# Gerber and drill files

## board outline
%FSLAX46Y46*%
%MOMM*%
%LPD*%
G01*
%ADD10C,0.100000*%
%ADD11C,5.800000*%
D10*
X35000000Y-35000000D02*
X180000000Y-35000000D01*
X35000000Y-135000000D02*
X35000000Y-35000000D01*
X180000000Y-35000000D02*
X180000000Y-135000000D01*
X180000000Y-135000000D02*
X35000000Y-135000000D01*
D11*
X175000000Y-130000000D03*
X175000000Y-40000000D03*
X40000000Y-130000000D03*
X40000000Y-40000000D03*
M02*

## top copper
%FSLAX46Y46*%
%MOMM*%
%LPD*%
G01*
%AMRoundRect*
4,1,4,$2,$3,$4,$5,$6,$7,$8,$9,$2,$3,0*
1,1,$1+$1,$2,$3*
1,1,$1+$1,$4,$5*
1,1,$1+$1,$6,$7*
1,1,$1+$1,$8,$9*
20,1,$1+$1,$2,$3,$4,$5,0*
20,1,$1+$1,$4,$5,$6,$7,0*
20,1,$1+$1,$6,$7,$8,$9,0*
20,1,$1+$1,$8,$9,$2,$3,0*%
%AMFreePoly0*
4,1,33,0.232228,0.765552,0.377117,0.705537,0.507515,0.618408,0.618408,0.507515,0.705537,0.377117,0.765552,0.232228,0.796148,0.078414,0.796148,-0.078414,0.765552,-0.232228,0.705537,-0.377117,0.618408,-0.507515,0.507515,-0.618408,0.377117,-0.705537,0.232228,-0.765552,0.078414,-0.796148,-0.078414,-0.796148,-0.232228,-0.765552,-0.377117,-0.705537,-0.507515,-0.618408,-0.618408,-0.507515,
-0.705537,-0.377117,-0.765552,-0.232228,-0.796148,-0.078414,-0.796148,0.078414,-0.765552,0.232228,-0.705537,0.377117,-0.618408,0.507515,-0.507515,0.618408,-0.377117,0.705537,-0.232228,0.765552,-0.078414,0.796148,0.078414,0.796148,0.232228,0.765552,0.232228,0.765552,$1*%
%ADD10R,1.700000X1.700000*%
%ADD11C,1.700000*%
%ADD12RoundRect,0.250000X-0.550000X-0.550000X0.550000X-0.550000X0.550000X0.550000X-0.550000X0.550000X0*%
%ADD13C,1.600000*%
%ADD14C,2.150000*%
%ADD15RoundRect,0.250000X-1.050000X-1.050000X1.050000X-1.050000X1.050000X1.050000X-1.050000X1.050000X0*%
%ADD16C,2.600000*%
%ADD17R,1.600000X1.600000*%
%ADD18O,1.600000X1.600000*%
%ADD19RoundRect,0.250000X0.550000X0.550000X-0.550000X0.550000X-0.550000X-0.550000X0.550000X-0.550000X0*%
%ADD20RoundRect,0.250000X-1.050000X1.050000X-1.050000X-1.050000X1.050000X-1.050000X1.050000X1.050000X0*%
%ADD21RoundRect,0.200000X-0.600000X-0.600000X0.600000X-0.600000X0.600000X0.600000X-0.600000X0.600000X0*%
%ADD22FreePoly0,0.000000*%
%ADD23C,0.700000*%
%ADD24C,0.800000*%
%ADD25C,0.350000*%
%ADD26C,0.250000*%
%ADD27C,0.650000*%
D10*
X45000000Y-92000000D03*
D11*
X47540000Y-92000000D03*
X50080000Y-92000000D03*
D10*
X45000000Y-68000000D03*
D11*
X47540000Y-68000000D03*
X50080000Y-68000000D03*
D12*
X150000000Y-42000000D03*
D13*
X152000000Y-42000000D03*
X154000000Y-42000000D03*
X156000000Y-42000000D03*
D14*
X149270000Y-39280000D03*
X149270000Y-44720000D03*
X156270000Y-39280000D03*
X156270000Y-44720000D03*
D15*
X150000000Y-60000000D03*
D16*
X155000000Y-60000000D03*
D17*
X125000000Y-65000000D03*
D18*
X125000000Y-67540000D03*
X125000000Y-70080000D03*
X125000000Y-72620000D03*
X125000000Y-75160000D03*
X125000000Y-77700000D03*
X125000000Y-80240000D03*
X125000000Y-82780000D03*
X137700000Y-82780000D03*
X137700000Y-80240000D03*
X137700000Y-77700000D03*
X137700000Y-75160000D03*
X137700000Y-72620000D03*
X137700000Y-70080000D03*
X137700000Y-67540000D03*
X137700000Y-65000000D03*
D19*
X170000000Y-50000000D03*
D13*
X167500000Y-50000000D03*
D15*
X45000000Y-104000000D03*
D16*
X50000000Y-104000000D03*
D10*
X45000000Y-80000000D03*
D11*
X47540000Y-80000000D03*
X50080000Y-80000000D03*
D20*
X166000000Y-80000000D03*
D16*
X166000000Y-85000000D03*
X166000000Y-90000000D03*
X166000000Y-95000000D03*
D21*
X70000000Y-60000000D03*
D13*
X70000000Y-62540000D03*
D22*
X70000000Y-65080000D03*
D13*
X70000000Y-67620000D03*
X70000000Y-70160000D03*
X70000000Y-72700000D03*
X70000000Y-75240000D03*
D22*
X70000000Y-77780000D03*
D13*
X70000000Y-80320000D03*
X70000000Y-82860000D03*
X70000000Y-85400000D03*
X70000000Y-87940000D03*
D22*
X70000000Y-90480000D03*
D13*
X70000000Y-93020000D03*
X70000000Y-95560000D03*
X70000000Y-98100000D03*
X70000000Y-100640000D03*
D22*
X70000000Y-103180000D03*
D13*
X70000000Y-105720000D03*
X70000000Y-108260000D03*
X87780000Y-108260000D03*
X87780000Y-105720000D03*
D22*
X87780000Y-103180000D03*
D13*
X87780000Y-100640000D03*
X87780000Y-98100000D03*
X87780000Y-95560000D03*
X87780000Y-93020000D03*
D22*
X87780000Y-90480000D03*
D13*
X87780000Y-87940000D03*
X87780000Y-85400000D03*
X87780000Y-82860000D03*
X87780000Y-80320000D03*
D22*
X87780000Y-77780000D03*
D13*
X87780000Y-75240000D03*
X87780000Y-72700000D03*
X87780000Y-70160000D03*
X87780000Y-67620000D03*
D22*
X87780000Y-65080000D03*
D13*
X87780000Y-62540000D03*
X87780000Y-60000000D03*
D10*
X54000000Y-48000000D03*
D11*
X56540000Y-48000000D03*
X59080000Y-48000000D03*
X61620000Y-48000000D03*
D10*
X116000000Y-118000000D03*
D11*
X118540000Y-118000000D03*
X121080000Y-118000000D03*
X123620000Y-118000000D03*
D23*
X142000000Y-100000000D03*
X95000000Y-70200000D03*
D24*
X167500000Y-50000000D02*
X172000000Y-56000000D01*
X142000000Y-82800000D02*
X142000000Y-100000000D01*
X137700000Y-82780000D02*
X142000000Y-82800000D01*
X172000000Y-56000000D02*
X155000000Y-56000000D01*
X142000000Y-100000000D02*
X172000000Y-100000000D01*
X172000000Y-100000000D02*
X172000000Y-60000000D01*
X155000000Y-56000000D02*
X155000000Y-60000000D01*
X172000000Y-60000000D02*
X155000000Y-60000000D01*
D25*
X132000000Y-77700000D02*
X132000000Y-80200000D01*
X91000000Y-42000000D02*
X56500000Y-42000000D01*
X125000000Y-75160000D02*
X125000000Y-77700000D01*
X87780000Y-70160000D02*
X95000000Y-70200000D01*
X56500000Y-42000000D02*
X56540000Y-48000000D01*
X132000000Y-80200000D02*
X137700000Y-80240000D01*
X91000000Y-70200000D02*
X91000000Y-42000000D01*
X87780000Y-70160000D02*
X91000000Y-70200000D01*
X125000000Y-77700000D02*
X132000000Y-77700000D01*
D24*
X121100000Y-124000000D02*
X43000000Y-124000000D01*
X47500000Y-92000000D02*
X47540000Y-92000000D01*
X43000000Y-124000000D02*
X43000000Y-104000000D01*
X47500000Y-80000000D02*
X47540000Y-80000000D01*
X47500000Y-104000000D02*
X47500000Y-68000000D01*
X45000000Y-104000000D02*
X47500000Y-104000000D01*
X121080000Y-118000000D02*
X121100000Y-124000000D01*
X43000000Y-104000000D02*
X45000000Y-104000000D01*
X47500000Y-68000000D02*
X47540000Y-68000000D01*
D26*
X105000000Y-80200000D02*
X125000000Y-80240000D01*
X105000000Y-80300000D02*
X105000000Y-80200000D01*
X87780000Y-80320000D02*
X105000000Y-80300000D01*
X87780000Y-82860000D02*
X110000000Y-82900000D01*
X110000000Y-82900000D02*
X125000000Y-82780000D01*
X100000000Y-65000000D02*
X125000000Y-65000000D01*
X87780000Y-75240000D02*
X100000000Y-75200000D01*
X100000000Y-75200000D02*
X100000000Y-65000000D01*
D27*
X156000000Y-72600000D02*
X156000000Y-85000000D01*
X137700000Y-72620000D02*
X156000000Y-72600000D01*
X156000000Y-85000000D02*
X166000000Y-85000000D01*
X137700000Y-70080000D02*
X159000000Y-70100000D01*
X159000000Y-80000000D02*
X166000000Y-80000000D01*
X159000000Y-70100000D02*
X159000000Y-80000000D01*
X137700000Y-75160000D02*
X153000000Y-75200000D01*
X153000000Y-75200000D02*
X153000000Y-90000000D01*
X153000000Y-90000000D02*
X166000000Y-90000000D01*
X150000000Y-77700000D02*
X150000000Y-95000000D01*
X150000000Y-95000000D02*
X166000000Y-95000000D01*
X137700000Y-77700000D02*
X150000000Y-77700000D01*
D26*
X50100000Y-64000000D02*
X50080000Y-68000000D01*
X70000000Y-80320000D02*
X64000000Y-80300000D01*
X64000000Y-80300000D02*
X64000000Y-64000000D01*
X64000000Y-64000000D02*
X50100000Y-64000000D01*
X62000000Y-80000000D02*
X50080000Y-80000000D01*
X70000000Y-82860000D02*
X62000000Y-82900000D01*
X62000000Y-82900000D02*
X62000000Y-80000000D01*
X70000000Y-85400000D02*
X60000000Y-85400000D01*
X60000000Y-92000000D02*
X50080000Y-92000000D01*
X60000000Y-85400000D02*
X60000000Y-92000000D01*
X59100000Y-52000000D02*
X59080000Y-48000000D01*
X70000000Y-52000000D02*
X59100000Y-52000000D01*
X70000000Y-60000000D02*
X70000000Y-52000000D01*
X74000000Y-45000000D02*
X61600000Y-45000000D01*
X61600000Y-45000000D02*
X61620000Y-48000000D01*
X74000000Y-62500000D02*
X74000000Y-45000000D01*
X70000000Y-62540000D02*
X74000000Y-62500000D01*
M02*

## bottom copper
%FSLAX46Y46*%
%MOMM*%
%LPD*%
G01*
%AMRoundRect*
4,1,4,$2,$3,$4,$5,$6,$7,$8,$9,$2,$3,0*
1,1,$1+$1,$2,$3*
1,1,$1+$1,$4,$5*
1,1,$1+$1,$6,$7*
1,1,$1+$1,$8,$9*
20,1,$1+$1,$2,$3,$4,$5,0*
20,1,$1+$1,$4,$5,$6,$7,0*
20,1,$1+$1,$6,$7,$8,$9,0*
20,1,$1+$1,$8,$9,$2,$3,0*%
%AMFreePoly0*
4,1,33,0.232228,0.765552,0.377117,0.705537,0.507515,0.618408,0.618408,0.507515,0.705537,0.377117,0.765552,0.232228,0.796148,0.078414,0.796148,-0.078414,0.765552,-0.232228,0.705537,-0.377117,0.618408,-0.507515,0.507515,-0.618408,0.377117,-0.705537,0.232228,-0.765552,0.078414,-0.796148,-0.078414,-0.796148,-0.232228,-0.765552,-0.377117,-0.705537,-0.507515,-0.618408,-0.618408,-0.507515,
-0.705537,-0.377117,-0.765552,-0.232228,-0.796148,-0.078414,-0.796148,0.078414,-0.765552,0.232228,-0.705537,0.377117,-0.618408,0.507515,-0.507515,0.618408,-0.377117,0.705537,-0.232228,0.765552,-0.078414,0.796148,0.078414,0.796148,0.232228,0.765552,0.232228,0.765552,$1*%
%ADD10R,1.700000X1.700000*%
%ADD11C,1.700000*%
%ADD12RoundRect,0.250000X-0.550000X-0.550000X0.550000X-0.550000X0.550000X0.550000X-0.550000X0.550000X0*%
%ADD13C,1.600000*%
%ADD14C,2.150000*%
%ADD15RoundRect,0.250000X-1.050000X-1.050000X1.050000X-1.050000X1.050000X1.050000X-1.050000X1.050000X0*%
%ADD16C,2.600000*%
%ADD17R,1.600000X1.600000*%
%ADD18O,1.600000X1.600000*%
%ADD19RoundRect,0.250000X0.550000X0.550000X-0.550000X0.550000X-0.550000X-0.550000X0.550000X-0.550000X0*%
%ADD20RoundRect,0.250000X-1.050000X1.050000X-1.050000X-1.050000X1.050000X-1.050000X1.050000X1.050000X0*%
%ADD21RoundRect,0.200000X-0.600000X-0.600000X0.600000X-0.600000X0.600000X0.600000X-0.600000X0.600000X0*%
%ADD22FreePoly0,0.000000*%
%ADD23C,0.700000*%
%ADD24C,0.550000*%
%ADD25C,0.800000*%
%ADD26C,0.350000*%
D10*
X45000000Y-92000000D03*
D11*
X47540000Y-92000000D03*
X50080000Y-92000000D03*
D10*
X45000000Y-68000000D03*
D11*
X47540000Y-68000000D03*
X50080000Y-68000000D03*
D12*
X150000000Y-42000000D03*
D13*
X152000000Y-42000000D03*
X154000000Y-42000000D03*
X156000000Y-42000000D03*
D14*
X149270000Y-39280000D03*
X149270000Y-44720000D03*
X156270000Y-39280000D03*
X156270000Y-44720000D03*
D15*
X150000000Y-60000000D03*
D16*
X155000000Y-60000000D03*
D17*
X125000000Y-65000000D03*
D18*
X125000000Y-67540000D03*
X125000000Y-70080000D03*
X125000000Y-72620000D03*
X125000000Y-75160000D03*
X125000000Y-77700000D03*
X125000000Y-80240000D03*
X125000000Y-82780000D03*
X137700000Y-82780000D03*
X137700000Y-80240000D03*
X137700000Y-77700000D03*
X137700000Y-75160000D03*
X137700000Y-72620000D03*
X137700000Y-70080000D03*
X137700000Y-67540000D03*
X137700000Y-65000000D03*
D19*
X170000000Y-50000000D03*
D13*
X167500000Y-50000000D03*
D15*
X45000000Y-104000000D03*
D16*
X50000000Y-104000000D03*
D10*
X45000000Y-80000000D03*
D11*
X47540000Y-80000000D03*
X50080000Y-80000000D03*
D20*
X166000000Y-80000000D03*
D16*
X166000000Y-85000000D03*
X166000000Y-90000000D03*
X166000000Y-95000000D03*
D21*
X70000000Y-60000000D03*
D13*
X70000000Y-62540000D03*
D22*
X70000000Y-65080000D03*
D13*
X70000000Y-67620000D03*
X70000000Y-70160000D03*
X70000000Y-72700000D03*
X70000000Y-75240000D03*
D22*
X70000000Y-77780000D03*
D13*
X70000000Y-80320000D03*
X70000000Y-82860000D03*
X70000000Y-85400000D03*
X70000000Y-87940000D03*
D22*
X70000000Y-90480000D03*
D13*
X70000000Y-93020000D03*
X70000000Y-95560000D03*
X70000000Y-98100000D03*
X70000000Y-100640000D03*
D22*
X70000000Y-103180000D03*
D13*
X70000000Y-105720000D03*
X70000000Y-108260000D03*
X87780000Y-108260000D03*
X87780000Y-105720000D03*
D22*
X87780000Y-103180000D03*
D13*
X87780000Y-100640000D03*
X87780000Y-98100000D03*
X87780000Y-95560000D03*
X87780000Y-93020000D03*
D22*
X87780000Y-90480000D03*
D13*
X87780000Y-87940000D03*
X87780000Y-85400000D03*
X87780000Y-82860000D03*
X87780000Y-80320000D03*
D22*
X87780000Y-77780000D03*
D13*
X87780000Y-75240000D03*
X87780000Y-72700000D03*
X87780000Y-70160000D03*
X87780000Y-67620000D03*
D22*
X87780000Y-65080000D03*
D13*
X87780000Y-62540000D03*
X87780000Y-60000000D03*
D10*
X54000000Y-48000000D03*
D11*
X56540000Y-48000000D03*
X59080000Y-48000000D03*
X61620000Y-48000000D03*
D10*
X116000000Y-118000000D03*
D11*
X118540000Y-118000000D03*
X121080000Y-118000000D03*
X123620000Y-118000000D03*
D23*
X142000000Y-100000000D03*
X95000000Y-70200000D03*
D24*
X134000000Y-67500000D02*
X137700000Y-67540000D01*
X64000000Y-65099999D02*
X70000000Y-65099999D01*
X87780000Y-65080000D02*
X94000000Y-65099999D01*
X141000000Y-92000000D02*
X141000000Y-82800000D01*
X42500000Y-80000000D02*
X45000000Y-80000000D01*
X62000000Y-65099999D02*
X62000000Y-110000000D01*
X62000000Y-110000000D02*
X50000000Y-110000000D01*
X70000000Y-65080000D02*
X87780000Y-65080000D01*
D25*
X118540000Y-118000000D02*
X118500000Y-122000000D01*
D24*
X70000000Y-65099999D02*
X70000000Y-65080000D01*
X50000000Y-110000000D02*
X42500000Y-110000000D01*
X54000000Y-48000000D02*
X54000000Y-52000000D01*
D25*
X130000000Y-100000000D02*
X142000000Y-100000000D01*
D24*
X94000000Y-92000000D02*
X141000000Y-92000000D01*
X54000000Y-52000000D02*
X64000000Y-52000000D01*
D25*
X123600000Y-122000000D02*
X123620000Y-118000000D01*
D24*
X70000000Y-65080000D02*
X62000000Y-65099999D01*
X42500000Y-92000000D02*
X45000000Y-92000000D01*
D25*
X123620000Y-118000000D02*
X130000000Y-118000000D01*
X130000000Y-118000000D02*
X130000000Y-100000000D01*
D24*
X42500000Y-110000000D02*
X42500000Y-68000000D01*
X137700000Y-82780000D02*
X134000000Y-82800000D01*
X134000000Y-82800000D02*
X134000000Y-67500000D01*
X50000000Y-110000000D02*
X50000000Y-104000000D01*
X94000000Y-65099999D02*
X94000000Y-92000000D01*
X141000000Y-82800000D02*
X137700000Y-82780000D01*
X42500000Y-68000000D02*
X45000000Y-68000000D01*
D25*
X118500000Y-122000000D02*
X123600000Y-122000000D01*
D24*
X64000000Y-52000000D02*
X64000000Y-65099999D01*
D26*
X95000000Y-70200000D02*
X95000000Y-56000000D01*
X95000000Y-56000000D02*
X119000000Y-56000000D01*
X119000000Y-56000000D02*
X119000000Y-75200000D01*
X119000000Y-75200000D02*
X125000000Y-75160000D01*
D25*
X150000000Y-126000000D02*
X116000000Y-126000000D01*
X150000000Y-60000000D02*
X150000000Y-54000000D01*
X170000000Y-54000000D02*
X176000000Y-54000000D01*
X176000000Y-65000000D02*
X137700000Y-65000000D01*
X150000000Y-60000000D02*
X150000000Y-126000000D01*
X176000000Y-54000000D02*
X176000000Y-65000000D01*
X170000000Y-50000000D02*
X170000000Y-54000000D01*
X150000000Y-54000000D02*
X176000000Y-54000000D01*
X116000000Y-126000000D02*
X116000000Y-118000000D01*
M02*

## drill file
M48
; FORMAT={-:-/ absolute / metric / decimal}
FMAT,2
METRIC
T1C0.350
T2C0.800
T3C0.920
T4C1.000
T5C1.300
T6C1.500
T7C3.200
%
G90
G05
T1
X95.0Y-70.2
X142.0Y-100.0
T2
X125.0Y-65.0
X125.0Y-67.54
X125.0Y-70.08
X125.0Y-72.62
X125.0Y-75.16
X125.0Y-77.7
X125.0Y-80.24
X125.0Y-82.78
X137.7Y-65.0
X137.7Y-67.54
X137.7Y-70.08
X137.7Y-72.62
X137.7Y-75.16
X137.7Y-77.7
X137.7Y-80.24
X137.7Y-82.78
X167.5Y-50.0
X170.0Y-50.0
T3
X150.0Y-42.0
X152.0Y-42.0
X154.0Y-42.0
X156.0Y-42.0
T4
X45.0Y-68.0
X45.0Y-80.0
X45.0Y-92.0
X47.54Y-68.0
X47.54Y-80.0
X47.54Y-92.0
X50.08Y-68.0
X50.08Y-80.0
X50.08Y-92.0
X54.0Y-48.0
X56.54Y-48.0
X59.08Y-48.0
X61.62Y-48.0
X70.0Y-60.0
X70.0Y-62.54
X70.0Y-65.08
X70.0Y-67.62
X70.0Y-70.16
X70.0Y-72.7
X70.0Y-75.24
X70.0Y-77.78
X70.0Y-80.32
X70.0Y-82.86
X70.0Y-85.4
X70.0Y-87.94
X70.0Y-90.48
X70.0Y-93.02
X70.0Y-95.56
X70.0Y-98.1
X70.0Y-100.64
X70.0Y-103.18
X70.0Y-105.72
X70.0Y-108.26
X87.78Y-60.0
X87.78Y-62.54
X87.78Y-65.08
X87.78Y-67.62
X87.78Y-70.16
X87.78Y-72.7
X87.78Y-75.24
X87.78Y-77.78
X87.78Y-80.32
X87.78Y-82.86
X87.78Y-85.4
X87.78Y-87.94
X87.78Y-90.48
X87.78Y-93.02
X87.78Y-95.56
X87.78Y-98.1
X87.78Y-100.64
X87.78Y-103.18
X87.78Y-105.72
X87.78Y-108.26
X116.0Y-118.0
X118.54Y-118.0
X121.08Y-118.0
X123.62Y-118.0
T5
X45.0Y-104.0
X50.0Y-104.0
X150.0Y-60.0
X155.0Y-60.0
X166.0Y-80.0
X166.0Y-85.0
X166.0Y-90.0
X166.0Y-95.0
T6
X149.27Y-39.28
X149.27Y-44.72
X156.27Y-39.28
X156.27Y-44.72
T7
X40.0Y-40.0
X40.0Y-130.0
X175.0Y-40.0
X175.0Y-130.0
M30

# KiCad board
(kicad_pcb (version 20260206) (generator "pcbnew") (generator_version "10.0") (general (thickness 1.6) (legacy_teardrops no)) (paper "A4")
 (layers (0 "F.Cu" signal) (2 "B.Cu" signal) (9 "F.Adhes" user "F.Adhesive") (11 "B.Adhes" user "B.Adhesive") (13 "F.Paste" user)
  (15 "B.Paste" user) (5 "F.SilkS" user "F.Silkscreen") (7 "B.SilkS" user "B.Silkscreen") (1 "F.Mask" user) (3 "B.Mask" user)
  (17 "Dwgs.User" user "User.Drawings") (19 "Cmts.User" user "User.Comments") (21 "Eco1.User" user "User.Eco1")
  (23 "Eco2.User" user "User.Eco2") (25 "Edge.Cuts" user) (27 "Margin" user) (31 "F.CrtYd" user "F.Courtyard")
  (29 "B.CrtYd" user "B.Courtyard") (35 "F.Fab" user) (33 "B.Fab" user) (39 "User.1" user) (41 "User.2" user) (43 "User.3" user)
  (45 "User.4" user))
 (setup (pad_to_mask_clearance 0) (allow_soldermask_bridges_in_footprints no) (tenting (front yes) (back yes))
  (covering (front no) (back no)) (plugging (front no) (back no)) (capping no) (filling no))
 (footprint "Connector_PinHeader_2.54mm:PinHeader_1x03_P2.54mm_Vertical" (layer "F.Cu") (at 45 92 90)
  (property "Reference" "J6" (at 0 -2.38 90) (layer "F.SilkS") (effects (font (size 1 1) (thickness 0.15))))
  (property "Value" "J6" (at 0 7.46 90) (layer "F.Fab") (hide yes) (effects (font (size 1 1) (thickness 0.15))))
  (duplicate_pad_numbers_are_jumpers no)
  (pad "1" thru_hole rect (at 0 0 90) (size 1.7 1.7) (drill 1) (layers "*.Cu" "*.Mask") (remove_unused_layers no) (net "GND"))
  (pad "2" thru_hole circle (at 0 2.54 90) (size 1.7 1.7) (drill 1) (layers "*.Cu" "*.Mask") (remove_unused_layers no) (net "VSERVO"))
  (pad "3" thru_hole circle (at 0 5.08 90) (size 1.7 1.7) (drill 1) (layers "*.Cu" "*.Mask") (remove_unused_layers no) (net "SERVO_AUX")))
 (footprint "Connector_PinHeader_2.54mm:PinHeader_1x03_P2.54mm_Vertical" (layer "F.Cu") (at 45 68 90)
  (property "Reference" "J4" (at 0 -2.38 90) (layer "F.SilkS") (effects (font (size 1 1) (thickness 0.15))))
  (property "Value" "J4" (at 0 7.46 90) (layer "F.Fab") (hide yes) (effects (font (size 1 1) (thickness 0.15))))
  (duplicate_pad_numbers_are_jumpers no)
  (pad "1" thru_hole rect (at 0 0 90) (size 1.7 1.7) (drill 1) (layers "*.Cu" "*.Mask") (remove_unused_layers no) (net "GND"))
  (pad "2" thru_hole circle (at 0 2.54 90) (size 1.7 1.7) (drill 1) (layers "*.Cu" "*.Mask") (remove_unused_layers no) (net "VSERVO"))
  (pad "3" thru_hole circle (at 0 5.08 90) (size 1.7 1.7) (drill 1) (layers "*.Cu" "*.Mask") (remove_unused_layers no) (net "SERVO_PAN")))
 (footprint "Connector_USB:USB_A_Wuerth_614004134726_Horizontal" (layer "F.Cu") (at 150 42)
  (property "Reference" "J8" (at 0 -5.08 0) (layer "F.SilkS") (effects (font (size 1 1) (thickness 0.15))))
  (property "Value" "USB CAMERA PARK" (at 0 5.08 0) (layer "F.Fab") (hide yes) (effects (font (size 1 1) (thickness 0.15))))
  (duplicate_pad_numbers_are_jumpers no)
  (pad "1" thru_hole roundrect (at 0 0) (size 1.6 1.6) (drill 0.92) (layers "*.Cu" "*.Mask") (remove_unused_layers no)
   (roundrect_rratio 0.15625) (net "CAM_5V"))
  (pad "2" thru_hole circle (at 2 0) (size 1.6 1.6) (drill 0.92) (layers "*.Cu" "*.Mask") (remove_unused_layers no) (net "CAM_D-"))
  (pad "3" thru_hole circle (at 4 0) (size 1.6 1.6) (drill 0.92) (layers "*.Cu" "*.Mask") (remove_unused_layers no) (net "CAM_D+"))
  (pad "4" thru_hole circle (at 6 0) (size 1.6 1.6) (drill 0.92) (layers "*.Cu" "*.Mask") (remove_unused_layers no) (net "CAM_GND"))
  (pad "SH" thru_hole circle (at -0.73 -2.72) (size 2.15 2.15) (drill 1.5) (layers "*.Cu" "*.Mask") (remove_unused_layers no))
  (pad "SH" thru_hole circle (at -0.73 2.72) (size 2.15 2.15) (drill 1.5) (layers "*.Cu" "*.Mask") (remove_unused_layers no))
  (pad "SH" thru_hole circle (at 6.27 -2.72) (size 2.15 2.15) (drill 1.5) (layers "*.Cu" "*.Mask") (remove_unused_layers no))
  (pad "SH" thru_hole circle (at 6.27 2.72) (size 2.15 2.15) (drill 1.5) (layers "*.Cu" "*.Mask") (remove_unused_layers no)))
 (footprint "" (layer "F.Cu") (at 175 130)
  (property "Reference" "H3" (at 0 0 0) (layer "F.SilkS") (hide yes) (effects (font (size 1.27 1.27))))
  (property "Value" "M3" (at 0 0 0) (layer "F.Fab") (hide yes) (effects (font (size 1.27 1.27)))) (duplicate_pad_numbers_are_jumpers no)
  (pad "" np_thru_hole circle (at 0 0) (size 5.8 5.8) (drill 3.2) (layers "Edge.Cuts")))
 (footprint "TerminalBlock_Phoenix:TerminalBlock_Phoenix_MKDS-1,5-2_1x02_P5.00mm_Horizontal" (layer "F.Cu") (at 150 60)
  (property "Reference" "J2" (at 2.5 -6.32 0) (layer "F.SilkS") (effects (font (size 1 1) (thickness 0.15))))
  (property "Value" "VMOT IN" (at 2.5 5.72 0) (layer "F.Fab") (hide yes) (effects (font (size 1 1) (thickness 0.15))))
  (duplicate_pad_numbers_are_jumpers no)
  (pad "1" thru_hole roundrect (at 0 0) (size 2.6 2.6) (drill 1.3) (layers "*.Cu" "*.Mask") (remove_unused_layers no)
   (roundrect_rratio 0.096154) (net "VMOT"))
  (pad "2" thru_hole circle (at 5 0) (size 2.6 2.6) (drill 1.3) (layers "*.Cu" "*.Mask") (remove_unused_layers no) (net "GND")))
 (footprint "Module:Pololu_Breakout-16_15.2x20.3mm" (layer "F.Cu") (at 125 65)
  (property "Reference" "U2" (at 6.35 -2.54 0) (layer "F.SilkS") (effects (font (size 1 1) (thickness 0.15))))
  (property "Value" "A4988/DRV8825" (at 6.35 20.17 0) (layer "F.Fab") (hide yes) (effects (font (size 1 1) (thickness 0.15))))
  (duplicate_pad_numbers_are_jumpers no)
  (pad "1" thru_hole rect (at 0 0) (size 1.6 1.6) (drill 0.8) (layers "*.Cu" "*.Mask") (remove_unused_layers no) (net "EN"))
  (pad "2" thru_hole oval (at 0 2.54) (size 1.6 1.6) (drill 0.8) (layers "*.Cu" "*.Mask") (remove_unused_layers no))
  (pad "3" thru_hole oval (at 0 5.08) (size 1.6 1.6) (drill 0.8) (layers "*.Cu" "*.Mask") (remove_unused_layers no))
  (pad "4" thru_hole oval (at 0 7.62) (size 1.6 1.6) (drill 0.8) (layers "*.Cu" "*.Mask") (remove_unused_layers no))
  (pad "5" thru_hole oval (at 0 10.16) (size 1.6 1.6) (drill 0.8) (layers "*.Cu" "*.Mask") (remove_unused_layers no) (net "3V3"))
  (pad "6" thru_hole oval (at 0 12.7) (size 1.6 1.6) (drill 0.8) (layers "*.Cu" "*.Mask") (remove_unused_layers no) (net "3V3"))
  (pad "7" thru_hole oval (at 0 15.24) (size 1.6 1.6) (drill 0.8) (layers "*.Cu" "*.Mask") (remove_unused_layers no) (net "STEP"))
  (pad "8" thru_hole oval (at 0 17.78) (size 1.6 1.6) (drill 0.8) (layers "*.Cu" "*.Mask") (remove_unused_layers no) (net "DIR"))
  (pad "9" thru_hole oval (at 12.7 17.78) (size 1.6 1.6) (drill 0.8) (layers "*.Cu" "*.Mask") (remove_unused_layers no) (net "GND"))
  (pad "10" thru_hole oval (at 12.7 15.24) (size 1.6 1.6) (drill 0.8) (layers "*.Cu" "*.Mask") (remove_unused_layers no) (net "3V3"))
  (pad "11" thru_hole oval (at 12.7 12.7) (size 1.6 1.6) (drill 0.8) (layers "*.Cu" "*.Mask") (remove_unused_layers no) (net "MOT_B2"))
  (pad "12" thru_hole oval (at 12.7 10.16) (size 1.6 1.6) (drill 0.8) (layers "*.Cu" "*.Mask") (remove_unused_layers no) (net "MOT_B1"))
  (pad "13" thru_hole oval (at 12.7 7.62) (size 1.6 1.6) (drill 0.8) (layers "*.Cu" "*.Mask") (remove_unused_layers no) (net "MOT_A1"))
  (pad "14" thru_hole oval (at 12.7 5.08) (size 1.6 1.6) (drill 0.8) (layers "*.Cu" "*.Mask") (remove_unused_layers no) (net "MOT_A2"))
  (pad "15" thru_hole oval (at 12.7 2.54) (size 1.6 1.6) (drill 0.8) (layers "*.Cu" "*.Mask") (remove_unused_layers no) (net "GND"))
  (pad "16" thru_hole oval (at 12.7 0) (size 1.6 1.6) (drill 0.8) (layers "*.Cu" "*.Mask") (remove_unused_layers no) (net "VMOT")))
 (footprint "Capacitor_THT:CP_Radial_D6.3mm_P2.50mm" (layer "F.Cu") (at 170 50 180)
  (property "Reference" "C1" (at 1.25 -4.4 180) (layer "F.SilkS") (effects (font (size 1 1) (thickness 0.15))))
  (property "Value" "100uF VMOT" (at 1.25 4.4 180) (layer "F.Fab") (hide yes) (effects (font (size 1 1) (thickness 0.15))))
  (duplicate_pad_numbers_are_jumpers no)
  (pad "1" thru_hole roundrect (at 0 0 180) (size 1.6 1.6) (drill 0.8) (layers "*.Cu" "*.Mask") (remove_unused_layers no)
   (roundrect_rratio 0.15625) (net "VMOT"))
  (pad "2" thru_hole circle (at 2.5 0 180) (size 1.6 1.6) (drill 0.8) (layers "*.Cu" "*.Mask") (remove_unused_layers no) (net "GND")))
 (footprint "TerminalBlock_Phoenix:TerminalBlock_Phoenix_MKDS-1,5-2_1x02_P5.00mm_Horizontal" (layer "F.Cu") (at 45 104)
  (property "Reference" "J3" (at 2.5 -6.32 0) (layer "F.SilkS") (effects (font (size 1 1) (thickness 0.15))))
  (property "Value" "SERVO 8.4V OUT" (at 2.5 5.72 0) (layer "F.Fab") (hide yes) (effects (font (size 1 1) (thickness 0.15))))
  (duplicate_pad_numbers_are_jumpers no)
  (pad "1" thru_hole roundrect (at 0 0) (size 2.6 2.6) (drill 1.3) (layers "*.Cu" "*.Mask") (remove_unused_layers no)
   (roundrect_rratio 0.096154) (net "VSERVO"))
  (pad "2" thru_hole circle (at 5 0) (size 2.6 2.6) (drill 1.3) (layers "*.Cu" "*.Mask") (remove_unused_layers no) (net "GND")))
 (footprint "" (layer "F.Cu") (at 175 40)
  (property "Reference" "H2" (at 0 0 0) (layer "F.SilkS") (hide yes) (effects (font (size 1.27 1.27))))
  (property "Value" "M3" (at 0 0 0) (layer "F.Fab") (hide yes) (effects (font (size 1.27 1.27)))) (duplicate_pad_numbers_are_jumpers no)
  (pad "" np_thru_hole circle (at 0 0) (size 5.8 5.8) (drill 3.2) (layers "Edge.Cuts")))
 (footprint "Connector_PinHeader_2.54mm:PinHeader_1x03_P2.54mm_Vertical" (layer "F.Cu") (at 45 80 90)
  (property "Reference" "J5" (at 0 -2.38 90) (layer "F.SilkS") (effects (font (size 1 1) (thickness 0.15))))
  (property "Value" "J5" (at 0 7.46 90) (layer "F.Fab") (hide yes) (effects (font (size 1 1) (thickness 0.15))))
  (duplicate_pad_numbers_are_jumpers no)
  (pad "1" thru_hole rect (at 0 0 90) (size 1.7 1.7) (drill 1) (layers "*.Cu" "*.Mask") (remove_unused_layers no) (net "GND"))
  (pad "2" thru_hole circle (at 0 2.54 90) (size 1.7 1.7) (drill 1) (layers "*.Cu" "*.Mask") (remove_unused_layers no) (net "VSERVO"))
  (pad "3" thru_hole circle (at 0 5.08 90) (size 1.7 1.7) (drill 1) (layers "*.Cu" "*.Mask") (remove_unused_layers no) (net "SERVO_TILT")))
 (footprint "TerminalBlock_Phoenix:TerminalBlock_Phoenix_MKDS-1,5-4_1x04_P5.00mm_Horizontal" (layer "F.Cu") (at 166 80 -90)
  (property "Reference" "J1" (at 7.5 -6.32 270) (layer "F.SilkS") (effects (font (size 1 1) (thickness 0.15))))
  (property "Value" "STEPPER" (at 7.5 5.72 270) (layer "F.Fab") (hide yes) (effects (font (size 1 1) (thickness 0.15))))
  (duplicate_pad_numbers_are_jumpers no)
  (pad "1" thru_hole roundrect (at 0 0 270) (size 2.6 2.6) (drill 1.3) (layers "*.Cu" "*.Mask") (remove_unused_layers no)
   (roundrect_rratio 0.096154) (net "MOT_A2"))
  (pad "2" thru_hole circle (at 5 0 270) (size 2.6 2.6) (drill 1.3) (layers "*.Cu" "*.Mask") (remove_unused_layers no) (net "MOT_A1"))
  (pad "3" thru_hole circle (at 10 0 270) (size 2.6 2.6) (drill 1.3) (layers "*.Cu" "*.Mask") (remove_unused_layers no) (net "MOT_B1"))
  (pad "4" thru_hole circle (at 15 0 270) (size 2.6 2.6) (drill 1.3) (layers "*.Cu" "*.Mask") (remove_unused_layers no) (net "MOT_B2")))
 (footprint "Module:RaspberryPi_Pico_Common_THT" (layer "F.Cu") (at 70 60)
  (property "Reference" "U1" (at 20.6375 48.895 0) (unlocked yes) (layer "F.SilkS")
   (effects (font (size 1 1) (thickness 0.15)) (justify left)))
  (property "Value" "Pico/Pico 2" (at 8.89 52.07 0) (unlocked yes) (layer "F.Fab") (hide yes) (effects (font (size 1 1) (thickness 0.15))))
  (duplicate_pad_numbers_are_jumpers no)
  (pad "1" thru_hole roundrect (at 0 0) (size 1.6 1.6) (drill 1) (layers "*.Cu" "*.Mask") (remove_unused_layers no) (roundrect_rratio 0.125)
   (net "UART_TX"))
  (pad "2" thru_hole circle (at 0 2.54) (size 1.6 1.6) (drill 1) (layers "*.Cu" "*.Mask") (remove_unused_layers no) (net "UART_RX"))
  (pad "3" thru_hole custom (at 0 5.08) (size 1.6 1.6) (drill 1) (layers "*.Cu" "*.Mask") (remove_unused_layers no) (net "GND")
   (options (clearance outline) (anchor circle)) (primitives))
  (pad "4" thru_hole circle (at 0 7.62) (size 1.6 1.6) (drill 1) (layers "*.Cu" "*.Mask") (remove_unused_layers no))
  (pad "5" thru_hole circle (at 0 10.16) (size 1.6 1.6) (drill 1) (layers "*.Cu" "*.Mask") (remove_unused_layers no))
  (pad "6" thru_hole circle (at 0 12.7) (size 1.6 1.6) (drill 1) (layers "*.Cu" "*.Mask") (remove_unused_layers no))
  (pad "7" thru_hole circle (at 0 15.24) (size 1.6 1.6) (drill 1) (layers "*.Cu" "*.Mask") (remove_unused_layers no))
  (pad "8" thru_hole custom (at 0 17.78) (size 1.6 1.6) (drill 1) (layers "*.Cu" "*.Mask") (remove_unused_layers no)
   (options (clearance outline) (anchor circle)) (primitives))
  (pad "9" thru_hole circle (at 0 20.32) (size 1.6 1.6) (drill 1) (layers "*.Cu" "*.Mask") (remove_unused_layers no) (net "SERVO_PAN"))
  (pad "10" thru_hole circle (at 0 22.86) (size 1.6 1.6) (drill 1) (layers "*.Cu" "*.Mask") (remove_unused_layers no) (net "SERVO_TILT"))
  (pad "11" thru_hole circle (at 0 25.4) (size 1.6 1.6) (drill 1) (layers "*.Cu" "*.Mask") (remove_unused_layers no) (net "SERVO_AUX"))
  (pad "12" thru_hole circle (at 0 27.94) (size 1.6 1.6) (drill 1) (layers "*.Cu" "*.Mask") (remove_unused_layers no))
  (pad "13" thru_hole custom (at 0 30.48) (size 1.6 1.6) (drill 1) (layers "*.Cu" "*.Mask") (remove_unused_layers no)
   (options (clearance outline) (anchor circle)) (primitives))
  (pad "14" thru_hole circle (at 0 33.02) (size 1.6 1.6) (drill 1) (layers "*.Cu" "*.Mask") (remove_unused_layers no))
  (pad "15" thru_hole circle (at 0 35.56) (size 1.6 1.6) (drill 1) (layers "*.Cu" "*.Mask") (remove_unused_layers no))
  (pad "16" thru_hole circle (at 0 38.1) (size 1.6 1.6) (drill 1) (layers "*.Cu" "*.Mask") (remove_unused_layers no))
  (pad "17" thru_hole circle (at 0 40.64) (size 1.6 1.6) (drill 1) (layers "*.Cu" "*.Mask") (remove_unused_layers no))
  (pad "18" thru_hole custom (at 0 43.18) (size 1.6 1.6) (drill 1) (layers "*.Cu" "*.Mask") (remove_unused_layers no)
   (options (clearance outline) (anchor circle)) (primitives))
  (pad "19" thru_hole circle (at 0 45.72) (size 1.6 1.6) (drill 1) (layers "*.Cu" "*.Mask") (remove_unused_layers no))
  (pad "20" thru_hole circle (at 0 48.26) (size 1.6 1.6) (drill 1) (layers "*.Cu" "*.Mask") (remove_unused_layers no))
  (pad "21" thru_hole circle (at 17.78 48.26) (size 1.6 1.6) (drill 1) (layers "*.Cu" "*.Mask") (remove_unused_layers no))
  (pad "22" thru_hole circle (at 17.78 45.72) (size 1.6 1.6) (drill 1) (layers "*.Cu" "*.Mask") (remove_unused_layers no))
  (pad "23" thru_hole custom (at 17.78 43.18) (size 1.6 1.6) (drill 1) (layers "*.Cu" "*.Mask") (remove_unused_layers no)
   (options (clearance outline) (anchor circle)) (primitives))
  (pad "24" thru_hole circle (at 17.78 40.64) (size 1.6 1.6) (drill 1) (layers "*.Cu" "*.Mask") (remove_unused_layers no))
  (pad "25" thru_hole circle (at 17.78 38.1) (size 1.6 1.6) (drill 1) (layers "*.Cu" "*.Mask") (remove_unused_layers no))
  (pad "26" thru_hole circle (at 17.78 35.56) (size 1.6 1.6) (drill 1) (layers "*.Cu" "*.Mask") (remove_unused_layers no))
  (pad "27" thru_hole circle (at 17.78 33.02) (size 1.6 1.6) (drill 1) (layers "*.Cu" "*.Mask") (remove_unused_layers no))
  (pad "28" thru_hole custom (at 17.78 30.48) (size 1.6 1.6) (drill 1) (layers "*.Cu" "*.Mask") (remove_unused_layers no)
   (options (clearance outline) (anchor circle)) (primitives))
  (pad "29" thru_hole circle (at 17.78 27.94) (size 1.6 1.6) (drill 1) (layers "*.Cu" "*.Mask") (remove_unused_layers no))
  (pad "30" thru_hole circle (at 17.78 25.4) (size 1.6 1.6) (drill 1) (layers "*.Cu" "*.Mask") (remove_unused_layers no))
  (pad "31" thru_hole circle (at 17.78 22.86) (size 1.6 1.6) (drill 1) (layers "*.Cu" "*.Mask") (remove_unused_layers no) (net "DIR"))
  (pad "32" thru_hole circle (at 17.78 20.32) (size 1.6 1.6) (drill 1) (layers "*.Cu" "*.Mask") (remove_unused_layers no) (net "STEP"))
  (pad "33" thru_hole custom (at 17.78 17.78) (size 1.6 1.6) (drill 1) (layers "*.Cu" "*.Mask") (remove_unused_layers no)
   (options (clearance outline) (anchor circle)) (primitives))
  (pad "34" thru_hole circle (at 17.78 15.24) (size 1.6 1.6) (drill 1) (layers "*.Cu" "*.Mask") (remove_unused_layers no) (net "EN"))
  (pad "35" thru_hole circle (at 17.78 12.7) (size 1.6 1.6) (drill 1) (layers "*.Cu" "*.Mask") (remove_unused_layers no))
  (pad "36" thru_hole circle (at 17.78 10.16) (size 1.6 1.6) (drill 1) (layers "*.Cu" "*.Mask") (remove_unused_layers no) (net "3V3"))
  (pad "37" thru_hole circle (at 17.78 7.62) (size 1.6 1.6) (drill 1) (layers "*.Cu" "*.Mask") (remove_unused_layers no))
  (pad "38" thru_hole custom (at 17.78 5.08) (size 1.6 1.6) (drill 1) (layers "*.Cu" "*.Mask") (remove_unused_layers no) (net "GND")
   (options (clearance outline) (anchor circle)) (primitives))
  (pad "39" thru_hole circle (at 17.78 2.54) (size 1.6 1.6) (drill 1) (layers "*.Cu" "*.Mask") (remove_unused_layers no))
  (pad "40" thru_hole circle (at 17.78 0) (size 1.6 1.6) (drill 1) (layers "*.Cu" "*.Mask") (remove_unused_layers no) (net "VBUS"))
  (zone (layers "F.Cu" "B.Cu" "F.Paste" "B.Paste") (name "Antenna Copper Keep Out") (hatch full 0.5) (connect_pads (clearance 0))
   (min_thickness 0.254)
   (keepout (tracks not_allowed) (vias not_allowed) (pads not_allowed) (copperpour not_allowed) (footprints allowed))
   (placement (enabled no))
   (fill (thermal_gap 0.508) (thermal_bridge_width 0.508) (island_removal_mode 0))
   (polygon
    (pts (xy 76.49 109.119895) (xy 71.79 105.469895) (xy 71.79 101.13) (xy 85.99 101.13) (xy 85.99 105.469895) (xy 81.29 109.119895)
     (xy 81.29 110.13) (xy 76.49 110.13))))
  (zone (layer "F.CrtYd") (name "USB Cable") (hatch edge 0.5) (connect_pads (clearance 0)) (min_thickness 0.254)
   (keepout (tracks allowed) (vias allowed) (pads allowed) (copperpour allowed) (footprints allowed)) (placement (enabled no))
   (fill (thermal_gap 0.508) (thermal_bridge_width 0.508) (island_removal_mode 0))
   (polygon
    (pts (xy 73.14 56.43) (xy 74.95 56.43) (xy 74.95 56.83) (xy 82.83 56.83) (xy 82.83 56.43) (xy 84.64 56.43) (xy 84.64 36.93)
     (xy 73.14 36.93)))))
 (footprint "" (layer "F.Cu") (at 40 130)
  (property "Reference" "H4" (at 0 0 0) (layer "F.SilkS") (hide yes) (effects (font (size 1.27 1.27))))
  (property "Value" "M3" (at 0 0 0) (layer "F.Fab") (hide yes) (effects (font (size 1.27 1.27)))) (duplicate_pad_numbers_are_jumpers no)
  (pad "" np_thru_hole circle (at 0 0) (size 5.8 5.8) (drill 3.2) (layers "Edge.Cuts")))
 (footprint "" (layer "F.Cu") (at 40 40)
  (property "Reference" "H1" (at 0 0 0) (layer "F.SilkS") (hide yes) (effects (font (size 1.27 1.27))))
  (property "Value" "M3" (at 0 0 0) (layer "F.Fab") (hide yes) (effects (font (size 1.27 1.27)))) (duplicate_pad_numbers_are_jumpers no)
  (pad "" np_thru_hole circle (at 0 0) (size 5.8 5.8) (drill 3.2) (layers "Edge.Cuts")))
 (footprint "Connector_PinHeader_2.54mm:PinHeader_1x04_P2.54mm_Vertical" (layer "F.Cu") (at 54 48 90)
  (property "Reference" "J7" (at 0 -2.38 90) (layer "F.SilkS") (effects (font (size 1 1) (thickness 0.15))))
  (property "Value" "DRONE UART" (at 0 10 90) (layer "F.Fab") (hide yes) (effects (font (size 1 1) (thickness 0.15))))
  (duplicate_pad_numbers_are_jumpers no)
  (pad "1" thru_hole rect (at 0 0 90) (size 1.7 1.7) (drill 1) (layers "*.Cu" "*.Mask") (remove_unused_layers no) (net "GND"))
  (pad "2" thru_hole circle (at 0 2.54 90) (size 1.7 1.7) (drill 1) (layers "*.Cu" "*.Mask") (remove_unused_layers no) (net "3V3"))
  (pad "3" thru_hole circle (at 0 5.08 90) (size 1.7 1.7) (drill 1) (layers "*.Cu" "*.Mask") (remove_unused_layers no) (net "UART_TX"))
  (pad "4" thru_hole circle (at 0 7.62 90) (size 1.7 1.7) (drill 1) (layers "*.Cu" "*.Mask") (remove_unused_layers no) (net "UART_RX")))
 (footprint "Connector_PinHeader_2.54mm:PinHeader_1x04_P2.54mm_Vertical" (layer "F.Cu") (at 116 118 90)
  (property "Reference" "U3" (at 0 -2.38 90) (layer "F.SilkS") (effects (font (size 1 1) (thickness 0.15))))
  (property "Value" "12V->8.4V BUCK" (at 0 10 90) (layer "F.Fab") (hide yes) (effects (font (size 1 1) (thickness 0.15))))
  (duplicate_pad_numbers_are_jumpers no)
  (pad "1" thru_hole rect (at 0 0 90) (size 1.7 1.7) (drill 1) (layers "*.Cu" "*.Mask") (remove_unused_layers no) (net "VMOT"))
  (pad "2" thru_hole circle (at 0 2.54 90) (size 1.7 1.7) (drill 1) (layers "*.Cu" "*.Mask") (remove_unused_layers no) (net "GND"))
  (pad "3" thru_hole circle (at 0 5.08 90) (size 1.7 1.7) (drill 1) (layers "*.Cu" "*.Mask") (remove_unused_layers no) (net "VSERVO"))
  (pad "4" thru_hole circle (at 0 7.62 90) (size 1.7 1.7) (drill 1) (layers "*.Cu" "*.Mask") (remove_unused_layers no) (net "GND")))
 (gr_line (start 35 35) (end 180 35) (stroke (width 0.1) (type default)) (layer "Edge.Cuts"))
 (gr_line (start 35 135) (end 35 35) (stroke (width 0.1) (type default)) (layer "Edge.Cuts"))
 (gr_line (start 180 35) (end 180 135) (stroke (width 0.1) (type default)) (layer "Edge.Cuts"))
 (gr_line (start 180 135) (end 35 135) (stroke (width 0.1) (type default)) (layer "Edge.Cuts"))
 (segment (start 167.5 50) (end 172 56) (width 0.8) (layer "F.Cu") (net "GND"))
 (segment (start 142 82.8) (end 142 100) (width 0.8) (layer "F.Cu") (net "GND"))
 (segment (start 137.7 82.78) (end 142 82.8) (width 0.8) (layer "F.Cu") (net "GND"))
 (segment (start 172 56) (end 155 56) (width 0.8) (layer "F.Cu") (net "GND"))
 (segment (start 142 100) (end 172 100) (width 0.8) (layer "F.Cu") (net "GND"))
 (segment (start 172 100) (end 172 60) (width 0.8) (layer "F.Cu") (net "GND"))
 (segment (start 155 56) (end 155 60) (width 0.8) (layer "F.Cu") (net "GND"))
 (segment (start 172 60) (end 155 60) (width 0.8) (layer "F.Cu") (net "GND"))
 (via (at 142 100) (size 0.7) (drill 0.35) (layers "F.Cu" "B.Cu") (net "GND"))
 (segment (start 134 67.5) (end 137.7 67.54) (width 0.55) (layer "B.Cu") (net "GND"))
 (segment (start 64 65.099999) (end 70 65.099999) (width 0.55) (layer "B.Cu") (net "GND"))
 (segment (start 87.78 65.08) (end 94 65.099999) (width 0.55) (layer "B.Cu") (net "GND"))
 (segment (start 141 92) (end 141 82.8) (width 0.55) (layer "B.Cu") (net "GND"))
 (segment (start 42.5 80) (end 45 80) (width 0.55) (layer "B.Cu") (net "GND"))
 (segment (start 62 65.099999) (end 62 110) (width 0.55) (layer "B.Cu") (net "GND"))
 (segment (start 62 110) (end 50 110) (width 0.55) (layer "B.Cu") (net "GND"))
 (segment (start 70 65.08) (end 87.78 65.08) (width 0.55) (layer "B.Cu") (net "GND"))
 (segment (start 118.54 118) (end 118.5 122) (width 0.8) (layer "B.Cu") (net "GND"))
 (segment (start 70 65.099999) (end 70 65.08) (width 0.55) (layer "B.Cu") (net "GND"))
 (segment (start 50 110) (end 42.5 110) (width 0.55) (layer "B.Cu") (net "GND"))
 (segment (start 54 48) (end 54 52) (width 0.55) (layer "B.Cu") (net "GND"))
 (segment (start 130 100) (end 142 100) (width 0.8) (layer "B.Cu") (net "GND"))
 (segment (start 94 92) (end 141 92) (width 0.55) (layer "B.Cu") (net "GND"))
 (segment (start 54 52) (end 64 52) (width 0.55) (layer "B.Cu") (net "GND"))
 (segment (start 123.6 122) (end 123.62 118) (width 0.8) (layer "B.Cu") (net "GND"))
 (segment (start 70 65.08) (end 62 65.099999) (width 0.55) (layer "B.Cu") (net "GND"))
 (segment (start 42.5 92) (end 45 92) (width 0.55) (layer "B.Cu") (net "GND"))
 (segment (start 123.62 118) (end 130 118) (width 0.8) (layer "B.Cu") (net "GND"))
 (segment (start 130 118) (end 130 100) (width 0.8) (layer "B.Cu") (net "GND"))
 (segment (start 42.5 110) (end 42.5 68) (width 0.55) (layer "B.Cu") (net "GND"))
 (segment (start 137.7 82.78) (end 134 82.8) (width 0.55) (layer "B.Cu") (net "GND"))
 (segment (start 134 82.8) (end 134 67.5) (width 0.55) (layer "B.Cu") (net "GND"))
 (segment (start 50 110) (end 50 104) (width 0.55) (layer "B.Cu") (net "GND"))
 (segment (start 94 65.099999) (end 94 92) (width 0.55) (layer "B.Cu") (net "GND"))
 (segment (start 141 82.8) (end 137.7 82.78) (width 0.55) (layer "B.Cu") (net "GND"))
 (segment (start 42.5 68) (end 45 68) (width 0.55) (layer "B.Cu") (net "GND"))
 (segment (start 118.5 122) (end 123.6 122) (width 0.8) (layer "B.Cu") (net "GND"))
 (segment (start 64 52) (end 64 65.099999) (width 0.55) (layer "B.Cu") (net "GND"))
 (segment (start 132 77.7) (end 132 80.2) (width 0.35) (layer "F.Cu") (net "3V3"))
 (segment (start 91 42) (end 56.5 42) (width 0.35) (layer "F.Cu") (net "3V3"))
 (segment (start 125 75.16) (end 125 77.7) (width 0.35) (layer "F.Cu") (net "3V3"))
 (segment (start 87.78 70.16) (end 95 70.2) (width 0.35) (layer "F.Cu") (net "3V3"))
 (segment (start 56.5 42) (end 56.54 48) (width 0.35) (layer "F.Cu") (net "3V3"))
 (segment (start 132 80.2) (end 137.7 80.24) (width 0.35) (layer "F.Cu") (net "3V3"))
 (segment (start 91 70.2) (end 91 42) (width 0.35) (layer "F.Cu") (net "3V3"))
 (segment (start 87.78 70.16) (end 91 70.2) (width 0.35) (layer "F.Cu") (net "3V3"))
 (segment (start 125 77.7) (end 132 77.7) (width 0.35) (layer "F.Cu") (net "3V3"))
 (via (at 95 70.2) (size 0.7) (drill 0.35) (layers "F.Cu" "B.Cu") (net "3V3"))
 (segment (start 95 70.2) (end 95 56) (width 0.35) (layer "B.Cu") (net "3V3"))
 (segment (start 95 56) (end 119 56) (width 0.35) (layer "B.Cu") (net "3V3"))
 (segment (start 119 56) (end 119 75.2) (width 0.35) (layer "B.Cu") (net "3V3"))
 (segment (start 119 75.2) (end 125 75.16) (width 0.35) (layer "B.Cu") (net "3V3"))
 (segment (start 121.1 124) (end 43 124) (width 0.8) (layer "F.Cu") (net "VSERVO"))
 (segment (start 47.5 92) (end 47.54 92) (width 0.8) (layer "F.Cu") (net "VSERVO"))
 (segment (start 43 124) (end 43 104) (width 0.8) (layer "F.Cu") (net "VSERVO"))
 (segment (start 47.5 80) (end 47.54 80) (width 0.8) (layer "F.Cu") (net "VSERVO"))
 (segment (start 47.5 104) (end 47.5 68) (width 0.8) (layer "F.Cu") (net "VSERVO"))
 (segment (start 45 104) (end 47.5 104) (width 0.8) (layer "F.Cu") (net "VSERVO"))
 (segment (start 121.08 118) (end 121.1 124) (width 0.8) (layer "F.Cu") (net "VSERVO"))
 (segment (start 43 104) (end 45 104) (width 0.8) (layer "F.Cu") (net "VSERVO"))
 (segment (start 47.5 68) (end 47.54 68) (width 0.8) (layer "F.Cu") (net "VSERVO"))
 (segment (start 150 126) (end 116 126) (width 0.8) (layer "B.Cu") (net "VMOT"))
 (segment (start 150 60) (end 150 54) (width 0.8) (layer "B.Cu") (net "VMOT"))
 (segment (start 170 54) (end 176 54) (width 0.8) (layer "B.Cu") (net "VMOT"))
 (segment (start 176 65) (end 137.7 65) (width 0.8) (layer "B.Cu") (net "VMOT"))
 (segment (start 150 60) (end 150 126) (width 0.8) (layer "B.Cu") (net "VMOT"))
 (segment (start 176 54) (end 176 65) (width 0.8) (layer "B.Cu") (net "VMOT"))
 (segment (start 170 50) (end 170 54) (width 0.8) (layer "B.Cu") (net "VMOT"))
 (segment (start 150 54) (end 176 54) (width 0.8) (layer "B.Cu") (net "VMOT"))
 (segment (start 116 126) (end 116 118) (width 0.8) (layer "B.Cu") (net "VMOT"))
 (segment (start 105 80.2) (end 125 80.24) (width 0.25) (layer "F.Cu") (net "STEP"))
 (segment (start 105 80.3) (end 105 80.2) (width 0.25) (layer "F.Cu") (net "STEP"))
 (segment (start 87.78 80.32) (end 105 80.3) (width 0.25) (layer "F.Cu") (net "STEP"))
 (segment (start 87.78 82.86) (end 110 82.9) (width 0.25) (layer "F.Cu") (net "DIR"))
 (segment (start 110 82.9) (end 125 82.78) (width 0.25) (layer "F.Cu") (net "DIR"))
 (segment (start 100 65) (end 125 65) (width 0.25) (layer "F.Cu") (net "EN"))
 (segment (start 87.78 75.24) (end 100 75.2) (width 0.25) (layer "F.Cu") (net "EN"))
 (segment (start 100 75.2) (end 100 65) (width 0.25) (layer "F.Cu") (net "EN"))
 (segment (start 156 72.6) (end 156 85) (width 0.65) (layer "F.Cu") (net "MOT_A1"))
 (segment (start 137.7 72.62) (end 156 72.6) (width 0.65) (layer "F.Cu") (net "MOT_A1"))
 (segment (start 156 85) (end 166 85) (width 0.65) (layer "F.Cu") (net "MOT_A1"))
 (segment (start 137.7 70.08) (end 159 70.1) (width 0.65) (layer "F.Cu") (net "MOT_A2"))
 (segment (start 159 80) (end 166 80) (width 0.65) (layer "F.Cu") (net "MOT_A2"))
 (segment (start 159 70.1) (end 159 80) (width 0.65) (layer "F.Cu") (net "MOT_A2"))
 (segment (start 137.7 75.16) (end 153 75.2) (width 0.65) (layer "F.Cu") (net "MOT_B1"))
 (segment (start 153 75.2) (end 153 90) (width 0.65) (layer "F.Cu") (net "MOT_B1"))
 (segment (start 153 90) (end 166 90) (width 0.65) (layer "F.Cu") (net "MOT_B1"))
 (segment (start 150 77.7) (end 150 95) (width 0.65) (layer "F.Cu") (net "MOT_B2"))
 (segment (start 150 95) (end 166 95) (width 0.65) (layer "F.Cu") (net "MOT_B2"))
 (segment (start 137.7 77.7) (end 150 77.7) (width 0.65) (layer "F.Cu") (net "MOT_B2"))
 (segment (start 50.1 64) (end 50.08 68) (width 0.25) (layer "F.Cu") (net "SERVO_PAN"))
 (segment (start 70 80.32) (end 64 80.3) (width 0.25) (layer "F.Cu") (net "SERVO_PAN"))
 (segment (start 64 80.3) (end 64 64) (width 0.25) (layer "F.Cu") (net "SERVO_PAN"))
 (segment (start 64 64) (end 50.1 64) (width 0.25) (layer "F.Cu") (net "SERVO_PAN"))
 (segment (start 62 80) (end 50.08 80) (width 0.25) (layer "F.Cu") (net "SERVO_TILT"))
 (segment (start 70 82.86) (end 62 82.9) (width 0.25) (layer "F.Cu") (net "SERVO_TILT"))
 (segment (start 62 82.9) (end 62 80) (width 0.25) (layer "F.Cu") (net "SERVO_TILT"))
 (segment (start 70 85.4) (end 60 85.4) (width 0.25) (layer "F.Cu") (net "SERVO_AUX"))
 (segment (start 60 92) (end 50.08 92) (width 0.25) (layer "F.Cu") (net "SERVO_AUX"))
 (segment (start 60 85.4) (end 60 92) (width 0.25) (layer "F.Cu") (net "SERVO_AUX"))
 (segment (start 59.1 52) (end 59.08 48) (width 0.25) (layer "F.Cu") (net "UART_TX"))
 (segment (start 70 52) (end 59.1 52) (width 0.25) (layer "F.Cu") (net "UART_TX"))
 (segment (start 70 60) (end 70 52) (width 0.25) (layer "F.Cu") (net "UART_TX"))
 (segment (start 74 45) (end 61.6 45) (width 0.25) (layer "F.Cu") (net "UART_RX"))
 (segment (start 61.6 45) (end 61.62 48) (width 0.25) (layer "F.Cu") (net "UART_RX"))
 (segment (start 74 62.5) (end 74 45) (width 0.25) (layer "F.Cu") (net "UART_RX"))
 (segment (start 70 62.54) (end 74 62.5) (width 0.25) (layer "F.Cu") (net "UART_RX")))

